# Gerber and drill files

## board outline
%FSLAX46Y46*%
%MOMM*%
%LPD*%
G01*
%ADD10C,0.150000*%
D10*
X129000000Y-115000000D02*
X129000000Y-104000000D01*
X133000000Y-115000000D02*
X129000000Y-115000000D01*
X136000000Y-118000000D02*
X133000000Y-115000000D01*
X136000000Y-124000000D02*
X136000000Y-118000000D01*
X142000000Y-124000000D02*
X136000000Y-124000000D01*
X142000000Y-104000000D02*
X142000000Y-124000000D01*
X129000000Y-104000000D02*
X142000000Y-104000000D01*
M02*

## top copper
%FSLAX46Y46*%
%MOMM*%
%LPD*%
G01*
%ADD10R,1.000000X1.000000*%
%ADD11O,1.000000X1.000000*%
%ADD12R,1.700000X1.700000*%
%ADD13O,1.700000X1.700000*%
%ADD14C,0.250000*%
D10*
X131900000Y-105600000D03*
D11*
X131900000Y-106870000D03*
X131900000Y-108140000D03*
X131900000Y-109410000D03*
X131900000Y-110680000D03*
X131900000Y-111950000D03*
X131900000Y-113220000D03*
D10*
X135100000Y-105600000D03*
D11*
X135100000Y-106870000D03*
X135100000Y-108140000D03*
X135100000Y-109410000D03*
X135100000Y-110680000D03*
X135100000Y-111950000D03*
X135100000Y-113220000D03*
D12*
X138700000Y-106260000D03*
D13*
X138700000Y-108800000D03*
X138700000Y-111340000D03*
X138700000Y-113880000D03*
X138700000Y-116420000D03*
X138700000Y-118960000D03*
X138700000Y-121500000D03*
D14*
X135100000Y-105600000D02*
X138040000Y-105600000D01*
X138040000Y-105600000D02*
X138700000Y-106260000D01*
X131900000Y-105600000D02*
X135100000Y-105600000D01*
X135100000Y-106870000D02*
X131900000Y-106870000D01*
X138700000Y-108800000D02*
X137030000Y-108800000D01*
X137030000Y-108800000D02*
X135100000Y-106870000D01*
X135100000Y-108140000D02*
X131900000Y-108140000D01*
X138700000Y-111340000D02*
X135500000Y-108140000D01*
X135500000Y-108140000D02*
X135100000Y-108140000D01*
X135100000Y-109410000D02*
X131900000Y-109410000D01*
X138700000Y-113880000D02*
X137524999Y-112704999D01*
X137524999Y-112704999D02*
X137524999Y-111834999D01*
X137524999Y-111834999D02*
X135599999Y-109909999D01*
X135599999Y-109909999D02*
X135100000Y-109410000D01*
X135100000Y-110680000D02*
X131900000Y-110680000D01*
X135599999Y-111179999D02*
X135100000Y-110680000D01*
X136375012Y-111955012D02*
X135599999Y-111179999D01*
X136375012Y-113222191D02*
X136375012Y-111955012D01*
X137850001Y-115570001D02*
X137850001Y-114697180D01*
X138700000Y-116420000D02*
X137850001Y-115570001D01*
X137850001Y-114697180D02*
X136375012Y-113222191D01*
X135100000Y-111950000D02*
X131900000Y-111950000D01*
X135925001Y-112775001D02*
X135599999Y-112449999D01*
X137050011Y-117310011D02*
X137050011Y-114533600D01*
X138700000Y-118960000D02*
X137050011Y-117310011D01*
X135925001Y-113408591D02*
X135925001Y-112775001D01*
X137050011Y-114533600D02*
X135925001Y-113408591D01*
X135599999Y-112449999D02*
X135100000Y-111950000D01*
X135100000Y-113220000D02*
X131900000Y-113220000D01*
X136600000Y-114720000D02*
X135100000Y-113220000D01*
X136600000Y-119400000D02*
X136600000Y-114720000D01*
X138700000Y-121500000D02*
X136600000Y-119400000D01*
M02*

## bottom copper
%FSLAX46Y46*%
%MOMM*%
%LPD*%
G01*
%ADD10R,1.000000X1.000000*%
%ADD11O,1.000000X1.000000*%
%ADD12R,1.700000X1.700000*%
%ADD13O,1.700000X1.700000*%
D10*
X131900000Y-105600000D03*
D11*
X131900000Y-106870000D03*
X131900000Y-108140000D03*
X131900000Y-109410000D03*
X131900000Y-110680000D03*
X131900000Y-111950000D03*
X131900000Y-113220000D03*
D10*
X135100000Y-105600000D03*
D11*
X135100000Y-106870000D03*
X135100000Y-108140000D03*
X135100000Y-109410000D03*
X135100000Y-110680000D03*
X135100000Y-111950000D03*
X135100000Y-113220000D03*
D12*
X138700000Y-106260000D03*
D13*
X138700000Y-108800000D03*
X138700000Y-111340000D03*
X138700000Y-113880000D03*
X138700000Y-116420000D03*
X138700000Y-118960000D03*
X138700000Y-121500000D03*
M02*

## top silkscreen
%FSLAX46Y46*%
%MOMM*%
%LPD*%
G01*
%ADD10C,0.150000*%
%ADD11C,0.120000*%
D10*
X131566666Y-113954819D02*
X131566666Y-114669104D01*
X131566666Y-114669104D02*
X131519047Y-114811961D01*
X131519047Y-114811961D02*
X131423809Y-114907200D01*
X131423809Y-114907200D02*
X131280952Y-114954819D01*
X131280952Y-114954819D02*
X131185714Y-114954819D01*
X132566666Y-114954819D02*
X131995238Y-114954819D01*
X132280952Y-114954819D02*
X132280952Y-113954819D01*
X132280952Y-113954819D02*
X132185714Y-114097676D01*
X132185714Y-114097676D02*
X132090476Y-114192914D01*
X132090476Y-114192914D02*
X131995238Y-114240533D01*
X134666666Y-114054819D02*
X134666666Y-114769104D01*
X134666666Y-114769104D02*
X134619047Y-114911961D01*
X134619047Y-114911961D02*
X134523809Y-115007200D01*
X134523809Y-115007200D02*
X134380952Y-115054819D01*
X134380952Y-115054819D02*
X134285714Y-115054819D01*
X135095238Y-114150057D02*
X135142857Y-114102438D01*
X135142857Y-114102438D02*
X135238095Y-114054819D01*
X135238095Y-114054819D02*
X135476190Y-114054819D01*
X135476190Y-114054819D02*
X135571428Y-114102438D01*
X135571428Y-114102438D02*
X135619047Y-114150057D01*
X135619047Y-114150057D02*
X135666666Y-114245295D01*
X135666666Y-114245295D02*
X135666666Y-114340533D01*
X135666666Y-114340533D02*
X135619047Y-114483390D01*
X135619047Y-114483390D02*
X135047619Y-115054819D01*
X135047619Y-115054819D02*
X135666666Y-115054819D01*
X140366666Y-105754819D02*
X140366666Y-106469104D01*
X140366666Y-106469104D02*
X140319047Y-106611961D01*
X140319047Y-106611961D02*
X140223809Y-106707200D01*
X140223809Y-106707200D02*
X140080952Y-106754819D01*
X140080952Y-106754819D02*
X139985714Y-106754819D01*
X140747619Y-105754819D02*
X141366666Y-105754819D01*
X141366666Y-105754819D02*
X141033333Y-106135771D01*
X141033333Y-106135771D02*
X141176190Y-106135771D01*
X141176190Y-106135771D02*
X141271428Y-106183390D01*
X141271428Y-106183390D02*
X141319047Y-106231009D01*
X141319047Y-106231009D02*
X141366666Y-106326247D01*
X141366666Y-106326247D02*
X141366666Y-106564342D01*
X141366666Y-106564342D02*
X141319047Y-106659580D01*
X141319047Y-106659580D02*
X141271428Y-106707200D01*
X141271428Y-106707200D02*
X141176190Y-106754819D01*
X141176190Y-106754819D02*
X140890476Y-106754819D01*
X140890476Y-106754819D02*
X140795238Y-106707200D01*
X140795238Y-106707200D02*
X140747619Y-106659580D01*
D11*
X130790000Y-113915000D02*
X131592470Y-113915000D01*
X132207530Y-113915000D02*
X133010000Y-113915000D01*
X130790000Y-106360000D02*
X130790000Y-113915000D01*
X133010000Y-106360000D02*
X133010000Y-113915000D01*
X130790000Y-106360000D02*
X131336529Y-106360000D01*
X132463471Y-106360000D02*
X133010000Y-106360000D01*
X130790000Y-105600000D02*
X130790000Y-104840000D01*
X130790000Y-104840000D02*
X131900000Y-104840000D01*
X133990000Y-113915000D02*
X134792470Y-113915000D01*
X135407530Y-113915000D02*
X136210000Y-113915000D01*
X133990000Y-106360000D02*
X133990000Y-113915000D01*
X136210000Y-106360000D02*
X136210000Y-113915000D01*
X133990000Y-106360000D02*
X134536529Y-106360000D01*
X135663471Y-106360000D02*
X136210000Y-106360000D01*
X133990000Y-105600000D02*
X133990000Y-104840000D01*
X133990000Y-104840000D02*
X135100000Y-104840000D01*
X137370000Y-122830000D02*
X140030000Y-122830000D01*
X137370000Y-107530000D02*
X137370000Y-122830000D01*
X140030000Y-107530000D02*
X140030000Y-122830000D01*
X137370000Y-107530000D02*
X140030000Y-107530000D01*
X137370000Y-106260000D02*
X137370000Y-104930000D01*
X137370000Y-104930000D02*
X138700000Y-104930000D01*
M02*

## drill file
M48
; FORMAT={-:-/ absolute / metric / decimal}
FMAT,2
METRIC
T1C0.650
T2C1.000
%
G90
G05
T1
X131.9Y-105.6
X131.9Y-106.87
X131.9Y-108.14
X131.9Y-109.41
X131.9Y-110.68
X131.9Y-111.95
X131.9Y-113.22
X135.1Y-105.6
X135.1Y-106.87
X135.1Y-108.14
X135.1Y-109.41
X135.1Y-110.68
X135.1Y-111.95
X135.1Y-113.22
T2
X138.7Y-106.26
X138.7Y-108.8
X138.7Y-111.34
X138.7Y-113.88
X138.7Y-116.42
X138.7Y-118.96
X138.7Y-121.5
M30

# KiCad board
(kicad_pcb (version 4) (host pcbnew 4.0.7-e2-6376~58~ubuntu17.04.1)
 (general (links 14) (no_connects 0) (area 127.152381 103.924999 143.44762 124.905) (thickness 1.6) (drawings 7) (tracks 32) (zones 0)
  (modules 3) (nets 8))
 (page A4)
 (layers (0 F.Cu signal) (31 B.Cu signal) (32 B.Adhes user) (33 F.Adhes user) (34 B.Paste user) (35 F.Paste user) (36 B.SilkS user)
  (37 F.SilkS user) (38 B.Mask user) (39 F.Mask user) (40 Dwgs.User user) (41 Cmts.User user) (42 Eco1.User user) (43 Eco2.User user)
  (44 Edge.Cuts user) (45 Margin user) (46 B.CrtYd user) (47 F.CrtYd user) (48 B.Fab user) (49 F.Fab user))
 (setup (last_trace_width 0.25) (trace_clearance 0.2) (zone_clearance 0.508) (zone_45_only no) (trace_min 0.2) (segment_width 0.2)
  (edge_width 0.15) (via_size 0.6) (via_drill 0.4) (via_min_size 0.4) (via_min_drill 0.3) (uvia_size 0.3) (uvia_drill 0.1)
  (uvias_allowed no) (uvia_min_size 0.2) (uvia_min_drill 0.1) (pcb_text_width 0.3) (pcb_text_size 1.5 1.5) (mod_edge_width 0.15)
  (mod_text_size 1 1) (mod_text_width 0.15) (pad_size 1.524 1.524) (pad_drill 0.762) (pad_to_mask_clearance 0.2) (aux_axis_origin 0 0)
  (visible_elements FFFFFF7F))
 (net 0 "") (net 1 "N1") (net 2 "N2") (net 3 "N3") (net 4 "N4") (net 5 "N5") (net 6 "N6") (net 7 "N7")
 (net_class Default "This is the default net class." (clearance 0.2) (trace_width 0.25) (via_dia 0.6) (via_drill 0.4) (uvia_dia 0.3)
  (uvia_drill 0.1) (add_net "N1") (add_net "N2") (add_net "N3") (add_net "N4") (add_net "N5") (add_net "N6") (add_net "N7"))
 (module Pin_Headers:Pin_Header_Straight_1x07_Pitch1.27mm (layer F.Cu) (at 131.9 105.6)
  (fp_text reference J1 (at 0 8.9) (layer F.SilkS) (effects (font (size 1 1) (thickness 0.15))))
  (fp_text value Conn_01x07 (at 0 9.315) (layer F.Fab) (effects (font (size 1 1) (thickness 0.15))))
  (fp_line (start -1.11 8.315) (end -0.30753 8.315) (layer F.SilkS) (width 0.12))
  (fp_line (start 0.30753 8.315) (end 1.11 8.315) (layer F.SilkS) (width 0.12))
  (fp_line (start -1.11 0.76) (end -1.11 8.315) (layer F.SilkS) (width 0.12))
  (fp_line (start 1.11 0.76) (end 1.11 8.315) (layer F.SilkS) (width 0.12))
  (fp_line (start -1.11 0.76) (end -0.563471 0.76) (layer F.SilkS) (width 0.12))
  (fp_line (start 0.563471 0.76) (end 1.11 0.76) (layer F.SilkS) (width 0.12))
  (fp_line (start -1.11 0) (end -1.11 -0.76) (layer F.SilkS) (width 0.12))
  (fp_line (start -1.11 -0.76) (end 0 -0.76) (layer F.SilkS) (width 0.12))
  (pad 1 thru_hole rect (at 0 0) (size 1 1) (drill 0.65) (layers *.Cu *.Mask) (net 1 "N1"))
  (pad 2 thru_hole oval (at 0 1.27) (size 1 1) (drill 0.65) (layers *.Cu *.Mask) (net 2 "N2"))
  (pad 3 thru_hole oval (at 0 2.54) (size 1 1) (drill 0.65) (layers *.Cu *.Mask) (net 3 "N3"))
  (pad 4 thru_hole oval (at 0 3.81) (size 1 1) (drill 0.65) (layers *.Cu *.Mask) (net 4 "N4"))
  (pad 5 thru_hole oval (at 0 5.08) (size 1 1) (drill 0.65) (layers *.Cu *.Mask) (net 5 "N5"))
  (pad 6 thru_hole oval (at 0 6.35) (size 1 1) (drill 0.65) (layers *.Cu *.Mask) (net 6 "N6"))
  (pad 7 thru_hole oval (at 0 7.62) (size 1 1) (drill 0.65) (layers *.Cu *.Mask) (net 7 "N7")))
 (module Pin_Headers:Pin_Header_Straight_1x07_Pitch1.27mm (layer F.Cu) (at 135.1 105.6)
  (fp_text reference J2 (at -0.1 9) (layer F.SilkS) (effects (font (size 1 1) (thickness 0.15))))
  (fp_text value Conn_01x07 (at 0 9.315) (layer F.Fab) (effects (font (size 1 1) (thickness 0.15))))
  (fp_line (start -1.11 8.315) (end -0.30753 8.315) (layer F.SilkS) (width 0.12))
  (fp_line (start 0.30753 8.315) (end 1.11 8.315) (layer F.SilkS) (width 0.12))
  (fp_line (start -1.11 0.76) (end -1.11 8.315) (layer F.SilkS) (width 0.12))
  (fp_line (start 1.11 0.76) (end 1.11 8.315) (layer F.SilkS) (width 0.12))
  (fp_line (start -1.11 0.76) (end -0.563471 0.76) (layer F.SilkS) (width 0.12))
  (fp_line (start 0.563471 0.76) (end 1.11 0.76) (layer F.SilkS) (width 0.12))
  (fp_line (start -1.11 0) (end -1.11 -0.76) (layer F.SilkS) (width 0.12))
  (fp_line (start -1.11 -0.76) (end 0 -0.76) (layer F.SilkS) (width 0.12))
  (pad 1 thru_hole rect (at 0 0) (size 1 1) (drill 0.65) (layers *.Cu *.Mask) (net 1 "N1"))
  (pad 2 thru_hole oval (at 0 1.27) (size 1 1) (drill 0.65) (layers *.Cu *.Mask) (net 2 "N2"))
  (pad 3 thru_hole oval (at 0 2.54) (size 1 1) (drill 0.65) (layers *.Cu *.Mask) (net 3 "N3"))
  (pad 4 thru_hole oval (at 0 3.81) (size 1 1) (drill 0.65) (layers *.Cu *.Mask) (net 4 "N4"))
  (pad 5 thru_hole oval (at 0 5.08) (size 1 1) (drill 0.65) (layers *.Cu *.Mask) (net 5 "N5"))
  (pad 6 thru_hole oval (at 0 6.35) (size 1 1) (drill 0.65) (layers *.Cu *.Mask) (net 6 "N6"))
  (pad 7 thru_hole oval (at 0 7.62) (size 1 1) (drill 0.65) (layers *.Cu *.Mask) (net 7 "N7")))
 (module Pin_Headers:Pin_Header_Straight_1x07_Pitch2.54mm (layer F.Cu) (at 138.7 106.26)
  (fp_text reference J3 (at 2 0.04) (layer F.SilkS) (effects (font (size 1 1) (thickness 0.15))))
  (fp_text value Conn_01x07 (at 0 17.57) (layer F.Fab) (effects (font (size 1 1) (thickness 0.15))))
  (fp_line (start -1.33 16.57) (end 1.33 16.57) (layer F.SilkS) (width 0.12))
  (fp_line (start -1.33 1.27) (end -1.33 16.57) (layer F.SilkS) (width 0.12))
  (fp_line (start 1.33 1.27) (end 1.33 16.57) (layer F.SilkS) (width 0.12))
  (fp_line (start -1.33 1.27) (end 1.33 1.27) (layer F.SilkS) (width 0.12))
  (fp_line (start -1.33 0) (end -1.33 -1.33) (layer F.SilkS) (width 0.12))
  (fp_line (start -1.33 -1.33) (end 0 -1.33) (layer F.SilkS) (width 0.12))
  (pad 1 thru_hole rect (at 0 0) (size 1.7 1.7) (drill 1) (layers *.Cu *.Mask) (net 1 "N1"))
  (pad 2 thru_hole oval (at 0 2.54) (size 1.7 1.7) (drill 1) (layers *.Cu *.Mask) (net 2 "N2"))
  (pad 3 thru_hole oval (at 0 5.08) (size 1.7 1.7) (drill 1) (layers *.Cu *.Mask) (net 3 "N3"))
  (pad 4 thru_hole oval (at 0 7.62) (size 1.7 1.7) (drill 1) (layers *.Cu *.Mask) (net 4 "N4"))
  (pad 5 thru_hole oval (at 0 10.16) (size 1.7 1.7) (drill 1) (layers *.Cu *.Mask) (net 5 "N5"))
  (pad 6 thru_hole oval (at 0 12.7) (size 1.7 1.7) (drill 1) (layers *.Cu *.Mask) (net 6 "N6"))
  (pad 7 thru_hole oval (at 0 15.24) (size 1.7 1.7) (drill 1) (layers *.Cu *.Mask) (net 7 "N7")))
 (gr_line (start 129 115) (end 129 104) (layer Edge.Cuts) (width 0.15))
 (gr_line (start 133 115) (end 129 115) (layer Edge.Cuts) (width 0.15))
 (gr_line (start 136 118) (end 133 115) (layer Edge.Cuts) (width 0.15))
 (gr_line (start 136 124) (end 136 118) (layer Edge.Cuts) (width 0.15))
 (gr_line (start 142 124) (end 136 124) (layer Edge.Cuts) (width 0.15))
 (gr_line (start 142 104) (end 142 124) (layer Edge.Cuts) (width 0.15))
 (gr_line (start 129 104) (end 142 104) (layer Edge.Cuts) (width 0.15))
 (segment (start 135.1 105.6) (end 138.04 105.6) (width 0.25) (layer F.Cu) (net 1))
 (segment (start 138.04 105.6) (end 138.7 106.26) (width 0.25) (layer F.Cu) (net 1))
 (segment (start 131.9 105.6) (end 135.1 105.6) (width 0.25) (layer F.Cu) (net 1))
 (segment (start 135.1 106.87) (end 131.9 106.87) (width 0.25) (layer F.Cu) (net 2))
 (segment (start 138.7 108.8) (end 137.03 108.8) (width 0.25) (layer F.Cu) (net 2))
 (segment (start 137.03 108.8) (end 135.1 106.87) (width 0.25) (layer F.Cu) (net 2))
 (segment (start 135.1 108.14) (end 131.9 108.14) (width 0.25) (layer F.Cu) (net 3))
 (segment (start 138.7 111.34) (end 135.5 108.14) (width 0.25) (layer F.Cu) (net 3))
 (segment (start 135.5 108.14) (end 135.1 108.14) (width 0.25) (layer F.Cu) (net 3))
 (segment (start 135.1 109.41) (end 131.9 109.41) (width 0.25) (layer F.Cu) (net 4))
 (segment (start 138.7 113.88) (end 137.524999 112.704999) (width 0.25) (layer F.Cu) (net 4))
 (segment (start 137.524999 112.704999) (end 137.524999 111.834999) (width 0.25) (layer F.Cu) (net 4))
 (segment (start 137.524999 111.834999) (end 135.599999 109.909999) (width 0.25) (layer F.Cu) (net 4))
 (segment (start 135.599999 109.909999) (end 135.1 109.41) (width 0.25) (layer F.Cu) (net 4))
 (segment (start 135.1 110.68) (end 131.9 110.68) (width 0.25) (layer F.Cu) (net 5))
 (segment (start 135.599999 111.179999) (end 135.1 110.68) (width 0.25) (layer F.Cu) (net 5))
 (segment (start 136.375012 111.955012) (end 135.599999 111.179999) (width 0.25) (layer F.Cu) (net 5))
 (segment (start 136.375012 113.222191) (end 136.375012 111.955012) (width 0.25) (layer F.Cu) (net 5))
 (segment (start 137.850001 115.570001) (end 137.850001 114.69718) (width 0.25) (layer F.Cu) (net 5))
 (segment (start 138.7 116.42) (end 137.850001 115.570001) (width 0.25) (layer F.Cu) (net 5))
 (segment (start 137.850001 114.69718) (end 136.375012 113.222191) (width 0.25) (layer F.Cu) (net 5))
 (segment (start 135.1 111.95) (end 131.9 111.95) (width 0.25) (layer F.Cu) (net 6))
 (segment (start 135.925001 112.775001) (end 135.599999 112.449999) (width 0.25) (layer F.Cu) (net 6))
 (segment (start 137.050011 117.310011) (end 137.050011 114.5336) (width 0.25) (layer F.Cu) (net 6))
 (segment (start 138.7 118.96) (end 137.050011 117.310011) (width 0.25) (layer F.Cu) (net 6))
 (segment (start 135.925001 113.408591) (end 135.925001 112.775001) (width 0.25) (layer F.Cu) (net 6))
 (segment (start 137.050011 114.5336) (end 135.925001 113.408591) (width 0.25) (layer F.Cu) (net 6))
 (segment (start 135.599999 112.449999) (end 135.1 111.95) (width 0.25) (layer F.Cu) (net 6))
 (segment (start 135.1 113.22) (end 131.9 113.22) (width 0.25) (layer F.Cu) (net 7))
 (segment (start 136.6 114.72) (end 135.1 113.22) (width 0.25) (layer F.Cu) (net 7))
 (segment (start 136.6 119.4) (end 136.6 114.72) (width 0.25) (layer F.Cu) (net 7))
 (segment (start 138.7 121.5) (end 136.6 119.4) (width 0.25) (layer F.Cu) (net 7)))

